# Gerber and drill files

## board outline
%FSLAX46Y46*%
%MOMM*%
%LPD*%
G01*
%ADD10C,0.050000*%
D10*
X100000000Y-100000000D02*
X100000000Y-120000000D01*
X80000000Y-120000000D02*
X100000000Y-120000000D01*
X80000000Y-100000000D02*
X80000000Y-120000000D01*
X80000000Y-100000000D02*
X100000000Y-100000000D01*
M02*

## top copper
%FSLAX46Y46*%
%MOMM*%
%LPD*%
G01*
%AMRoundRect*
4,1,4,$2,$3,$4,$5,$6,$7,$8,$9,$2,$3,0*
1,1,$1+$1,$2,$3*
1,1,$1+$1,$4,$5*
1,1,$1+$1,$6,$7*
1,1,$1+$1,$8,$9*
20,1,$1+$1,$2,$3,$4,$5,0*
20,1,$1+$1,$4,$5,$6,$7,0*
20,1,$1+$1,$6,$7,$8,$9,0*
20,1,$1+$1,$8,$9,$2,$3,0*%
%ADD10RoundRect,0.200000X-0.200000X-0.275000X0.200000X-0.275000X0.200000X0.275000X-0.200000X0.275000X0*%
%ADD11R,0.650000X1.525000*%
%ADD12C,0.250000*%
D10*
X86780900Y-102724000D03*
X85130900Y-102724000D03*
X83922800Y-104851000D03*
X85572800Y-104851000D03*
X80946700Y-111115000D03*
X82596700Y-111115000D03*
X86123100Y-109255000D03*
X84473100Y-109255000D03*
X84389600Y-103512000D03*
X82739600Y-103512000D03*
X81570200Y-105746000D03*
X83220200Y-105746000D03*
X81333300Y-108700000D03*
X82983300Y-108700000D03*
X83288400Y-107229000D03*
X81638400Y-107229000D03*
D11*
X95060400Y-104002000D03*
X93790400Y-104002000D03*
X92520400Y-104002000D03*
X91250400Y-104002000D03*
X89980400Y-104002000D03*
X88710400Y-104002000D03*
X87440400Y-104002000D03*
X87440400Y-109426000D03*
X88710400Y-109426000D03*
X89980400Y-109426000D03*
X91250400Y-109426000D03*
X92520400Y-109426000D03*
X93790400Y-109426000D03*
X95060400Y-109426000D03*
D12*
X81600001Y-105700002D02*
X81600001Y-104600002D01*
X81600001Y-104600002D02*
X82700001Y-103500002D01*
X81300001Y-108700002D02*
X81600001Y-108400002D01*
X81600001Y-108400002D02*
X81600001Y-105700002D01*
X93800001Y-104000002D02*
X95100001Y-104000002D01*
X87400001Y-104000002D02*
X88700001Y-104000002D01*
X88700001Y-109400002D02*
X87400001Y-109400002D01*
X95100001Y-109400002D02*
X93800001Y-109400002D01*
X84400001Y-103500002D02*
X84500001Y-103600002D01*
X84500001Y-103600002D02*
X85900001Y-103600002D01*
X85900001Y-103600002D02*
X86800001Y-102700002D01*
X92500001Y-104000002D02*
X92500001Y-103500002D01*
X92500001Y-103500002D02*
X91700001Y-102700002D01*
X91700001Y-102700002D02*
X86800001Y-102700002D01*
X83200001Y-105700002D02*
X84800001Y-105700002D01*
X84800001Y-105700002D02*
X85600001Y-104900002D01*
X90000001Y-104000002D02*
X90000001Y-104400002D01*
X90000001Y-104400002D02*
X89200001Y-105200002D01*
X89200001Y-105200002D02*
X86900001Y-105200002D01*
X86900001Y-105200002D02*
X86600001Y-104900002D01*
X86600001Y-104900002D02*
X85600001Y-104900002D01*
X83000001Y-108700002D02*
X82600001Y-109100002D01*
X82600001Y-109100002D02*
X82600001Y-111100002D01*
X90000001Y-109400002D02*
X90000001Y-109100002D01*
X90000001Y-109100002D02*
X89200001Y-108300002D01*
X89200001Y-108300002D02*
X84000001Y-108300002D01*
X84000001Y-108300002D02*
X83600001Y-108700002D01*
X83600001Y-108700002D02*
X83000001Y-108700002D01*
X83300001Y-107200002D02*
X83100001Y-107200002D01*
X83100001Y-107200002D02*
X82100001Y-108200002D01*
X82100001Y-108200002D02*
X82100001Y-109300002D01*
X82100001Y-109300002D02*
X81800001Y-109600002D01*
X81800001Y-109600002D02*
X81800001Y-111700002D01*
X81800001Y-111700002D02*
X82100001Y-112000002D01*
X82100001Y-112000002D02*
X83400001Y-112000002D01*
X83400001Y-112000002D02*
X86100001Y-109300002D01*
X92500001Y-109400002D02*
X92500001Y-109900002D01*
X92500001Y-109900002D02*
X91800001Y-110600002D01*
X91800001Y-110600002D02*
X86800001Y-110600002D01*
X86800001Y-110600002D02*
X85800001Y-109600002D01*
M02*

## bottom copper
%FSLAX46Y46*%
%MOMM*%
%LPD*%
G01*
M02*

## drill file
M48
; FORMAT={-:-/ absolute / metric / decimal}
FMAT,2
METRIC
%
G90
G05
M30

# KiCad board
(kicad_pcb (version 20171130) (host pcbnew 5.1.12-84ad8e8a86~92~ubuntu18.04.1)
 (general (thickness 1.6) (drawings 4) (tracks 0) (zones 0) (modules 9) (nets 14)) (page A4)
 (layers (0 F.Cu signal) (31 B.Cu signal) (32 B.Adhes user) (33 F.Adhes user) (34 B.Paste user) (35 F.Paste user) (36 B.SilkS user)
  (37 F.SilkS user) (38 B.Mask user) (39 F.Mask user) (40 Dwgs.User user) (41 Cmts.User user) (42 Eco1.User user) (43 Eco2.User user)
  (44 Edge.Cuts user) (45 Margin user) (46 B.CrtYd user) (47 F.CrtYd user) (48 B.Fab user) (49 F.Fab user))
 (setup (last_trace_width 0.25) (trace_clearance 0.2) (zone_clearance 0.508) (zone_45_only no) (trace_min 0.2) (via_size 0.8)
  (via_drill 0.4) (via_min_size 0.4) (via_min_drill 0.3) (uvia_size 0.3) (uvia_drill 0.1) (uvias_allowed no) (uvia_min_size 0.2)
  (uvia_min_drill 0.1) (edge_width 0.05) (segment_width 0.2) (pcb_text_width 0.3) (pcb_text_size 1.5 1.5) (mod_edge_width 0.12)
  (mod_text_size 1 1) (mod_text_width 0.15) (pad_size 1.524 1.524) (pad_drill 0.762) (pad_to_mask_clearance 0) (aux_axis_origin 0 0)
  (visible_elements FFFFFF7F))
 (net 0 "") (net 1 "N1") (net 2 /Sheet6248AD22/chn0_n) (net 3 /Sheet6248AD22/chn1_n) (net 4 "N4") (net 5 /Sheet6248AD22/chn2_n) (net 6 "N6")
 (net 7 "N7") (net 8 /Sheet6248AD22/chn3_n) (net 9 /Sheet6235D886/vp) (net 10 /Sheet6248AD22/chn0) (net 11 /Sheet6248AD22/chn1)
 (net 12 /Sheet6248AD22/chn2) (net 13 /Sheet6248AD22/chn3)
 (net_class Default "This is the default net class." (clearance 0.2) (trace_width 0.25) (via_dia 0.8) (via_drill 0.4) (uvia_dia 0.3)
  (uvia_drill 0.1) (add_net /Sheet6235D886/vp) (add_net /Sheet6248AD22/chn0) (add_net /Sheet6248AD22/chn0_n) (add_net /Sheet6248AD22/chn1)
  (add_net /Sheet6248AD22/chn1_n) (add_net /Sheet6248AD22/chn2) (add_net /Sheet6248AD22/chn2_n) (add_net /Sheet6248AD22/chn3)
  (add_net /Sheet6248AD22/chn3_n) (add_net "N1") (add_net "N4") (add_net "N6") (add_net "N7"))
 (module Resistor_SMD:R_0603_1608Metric (layer F.Cu) (at 85.955900 102.724000)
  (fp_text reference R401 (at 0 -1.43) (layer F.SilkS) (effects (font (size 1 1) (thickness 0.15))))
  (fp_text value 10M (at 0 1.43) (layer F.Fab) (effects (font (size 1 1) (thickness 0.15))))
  (pad 2 smd roundrect (at 0.825 0) (size 0.8 0.95) (layers F.Cu F.Mask F.Paste) (roundrect_rratio 0.25) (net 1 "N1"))
  (pad 1 smd roundrect (at -0.825 0) (size 0.8 0.95) (layers F.Cu F.Mask F.Paste) (roundrect_rratio 0.25) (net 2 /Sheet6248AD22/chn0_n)))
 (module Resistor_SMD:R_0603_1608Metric (layer F.Cu) (at 84.747800 104.851000)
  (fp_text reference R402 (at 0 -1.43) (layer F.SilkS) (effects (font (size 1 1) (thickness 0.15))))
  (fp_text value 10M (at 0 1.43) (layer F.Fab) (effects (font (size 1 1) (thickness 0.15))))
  (pad 1 smd roundrect (at -0.825 0) (size 0.8 0.95) (layers F.Cu F.Mask F.Paste) (roundrect_rratio 0.25) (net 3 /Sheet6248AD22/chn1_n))
  (pad 2 smd roundrect (at 0.825 0) (size 0.8 0.95) (layers F.Cu F.Mask F.Paste) (roundrect_rratio 0.25) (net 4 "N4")))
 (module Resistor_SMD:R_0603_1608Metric (layer F.Cu) (at 81.771700 111.115000)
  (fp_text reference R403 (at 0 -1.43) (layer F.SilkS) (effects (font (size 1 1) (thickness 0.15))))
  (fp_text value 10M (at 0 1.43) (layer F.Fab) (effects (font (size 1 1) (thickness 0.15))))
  (pad 1 smd roundrect (at -0.825 0) (size 0.8 0.95) (layers F.Cu F.Mask F.Paste) (roundrect_rratio 0.25) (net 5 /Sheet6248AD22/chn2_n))
  (pad 2 smd roundrect (at 0.825 0) (size 0.8 0.95) (layers F.Cu F.Mask F.Paste) (roundrect_rratio 0.25) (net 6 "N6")))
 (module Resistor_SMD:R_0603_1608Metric (layer F.Cu) (at 85.298100 109.255000)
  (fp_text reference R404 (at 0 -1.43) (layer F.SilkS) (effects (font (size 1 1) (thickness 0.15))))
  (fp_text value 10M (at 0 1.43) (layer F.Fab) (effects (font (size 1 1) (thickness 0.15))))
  (pad 2 smd roundrect (at 0.825 0) (size 0.8 0.95) (layers F.Cu F.Mask F.Paste) (roundrect_rratio 0.25) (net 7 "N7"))
  (pad 1 smd roundrect (at -0.825 0) (size 0.8 0.95) (layers F.Cu F.Mask F.Paste) (roundrect_rratio 0.25) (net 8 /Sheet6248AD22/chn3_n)))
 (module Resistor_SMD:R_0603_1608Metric (layer F.Cu) (at 83.564600 103.512000)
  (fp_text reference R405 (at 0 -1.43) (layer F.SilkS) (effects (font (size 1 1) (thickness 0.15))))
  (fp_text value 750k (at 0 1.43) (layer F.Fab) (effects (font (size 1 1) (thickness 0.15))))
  (pad 2 smd roundrect (at 0.825 0) (size 0.8 0.95) (layers F.Cu F.Mask F.Paste) (roundrect_rratio 0.25) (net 1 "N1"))
  (pad 1 smd roundrect (at -0.825 0) (size 0.8 0.95) (layers F.Cu F.Mask F.Paste) (roundrect_rratio 0.25) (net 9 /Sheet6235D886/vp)))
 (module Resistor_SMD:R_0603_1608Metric (layer F.Cu) (at 82.395200 105.746000)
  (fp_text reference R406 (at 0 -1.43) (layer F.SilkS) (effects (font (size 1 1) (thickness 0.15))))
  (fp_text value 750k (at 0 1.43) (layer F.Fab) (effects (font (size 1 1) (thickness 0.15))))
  (pad 1 smd roundrect (at -0.825 0) (size 0.8 0.95) (layers F.Cu F.Mask F.Paste) (roundrect_rratio 0.25) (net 9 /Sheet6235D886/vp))
  (pad 2 smd roundrect (at 0.825 0) (size 0.8 0.95) (layers F.Cu F.Mask F.Paste) (roundrect_rratio 0.25) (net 4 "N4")))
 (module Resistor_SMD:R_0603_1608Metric (layer F.Cu) (at 82.158300 108.700000)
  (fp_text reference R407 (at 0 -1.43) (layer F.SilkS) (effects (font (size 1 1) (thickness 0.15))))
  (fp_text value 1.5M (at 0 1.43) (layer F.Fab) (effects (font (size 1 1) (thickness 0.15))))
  (pad 1 smd roundrect (at -0.825 0) (size 0.8 0.95) (layers F.Cu F.Mask F.Paste) (roundrect_rratio 0.25) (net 9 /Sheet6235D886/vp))
  (pad 2 smd roundrect (at 0.825 0) (size 0.8 0.95) (layers F.Cu F.Mask F.Paste) (roundrect_rratio 0.25) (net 6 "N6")))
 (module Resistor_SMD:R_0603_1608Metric (layer F.Cu) (at 82.463400 107.229000)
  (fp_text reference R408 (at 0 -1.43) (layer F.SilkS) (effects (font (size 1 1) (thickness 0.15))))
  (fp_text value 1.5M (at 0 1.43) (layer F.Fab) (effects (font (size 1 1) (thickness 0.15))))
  (pad 2 smd roundrect (at 0.825 0) (size 0.8 0.95) (layers F.Cu F.Mask F.Paste) (roundrect_rratio 0.25) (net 7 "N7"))
  (pad 1 smd roundrect (at -0.825 0) (size 0.8 0.95) (layers F.Cu F.Mask F.Paste) (roundrect_rratio 0.25) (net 9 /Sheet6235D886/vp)))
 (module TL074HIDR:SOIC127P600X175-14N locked (layer F.Cu) (at 91.250400 106.714000 270.000000)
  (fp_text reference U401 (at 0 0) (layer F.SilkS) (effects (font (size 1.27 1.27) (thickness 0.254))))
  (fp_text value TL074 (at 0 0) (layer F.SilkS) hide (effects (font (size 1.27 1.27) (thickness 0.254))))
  (pad 1 smd rect (at -2.712 -3.81) (size 0.65 1.525) (layers F.Cu F.Mask F.Paste) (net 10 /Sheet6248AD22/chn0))
  (pad 2 smd rect (at -2.712 -2.54) (size 0.65 1.525) (layers F.Cu F.Mask F.Paste) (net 10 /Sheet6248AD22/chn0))
  (pad 3 smd rect (at -2.712 -1.27) (size 0.65 1.525) (layers F.Cu F.Mask F.Paste) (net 1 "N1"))
  (pad 4 smd rect (at -2.712 0) (size 0.65 1.525) (layers F.Cu F.Mask F.Paste))
  (pad 5 smd rect (at -2.712 1.27) (size 0.65 1.525) (layers F.Cu F.Mask F.Paste) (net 4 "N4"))
  (pad 6 smd rect (at -2.712 2.54) (size 0.65 1.525) (layers F.Cu F.Mask F.Paste) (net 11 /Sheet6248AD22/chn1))
  (pad 7 smd rect (at -2.712 3.81) (size 0.65 1.525) (layers F.Cu F.Mask F.Paste) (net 11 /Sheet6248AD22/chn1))
  (pad 8 smd rect (at 2.712 3.81) (size 0.65 1.525) (layers F.Cu F.Mask F.Paste) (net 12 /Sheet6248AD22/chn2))
  (pad 9 smd rect (at 2.712 2.54) (size 0.65 1.525) (layers F.Cu F.Mask F.Paste) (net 12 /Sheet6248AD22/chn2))
  (pad 10 smd rect (at 2.712 1.27) (size 0.65 1.525) (layers F.Cu F.Mask F.Paste) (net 6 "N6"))
  (pad 11 smd rect (at 2.712 0) (size 0.65 1.525) (layers F.Cu F.Mask F.Paste))
  (pad 12 smd rect (at 2.712 -1.27) (size 0.65 1.525) (layers F.Cu F.Mask F.Paste) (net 7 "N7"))
  (pad 13 smd rect (at 2.712 -2.54) (size 0.65 1.525) (layers F.Cu F.Mask F.Paste) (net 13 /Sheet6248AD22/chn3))
  (pad 14 smd rect (at 2.712 -3.81) (size 0.65 1.525) (layers F.Cu F.Mask F.Paste) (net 13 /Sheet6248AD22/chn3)))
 (gr_line (start 100 100) (end 100 120) (layer Edge.Cuts) (width 0.05))
 (gr_line (start 80 120) (end 100 120) (layer Edge.Cuts) (width 0.05))
 (gr_line (start 80 100) (end 80 120) (layer Edge.Cuts) (width 0.05))
 (gr_line (start 80 100) (end 100 100) (layer Edge.Cuts) (width 0.05))
 (segment (start 81.600001 105.700002) (end 81.600001 104.600002) (width 0.250000) (layer F.Cu) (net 9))
 (segment (start 81.600001 104.600002) (end 82.700001 103.500002) (width 0.250000) (layer F.Cu) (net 9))
 (segment (start 81.300001 108.700002) (end 81.600001 108.400002) (width 0.250000) (layer F.Cu) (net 9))
 (segment (start 81.600001 108.400002) (end 81.600001 105.700002) (width 0.250000) (layer F.Cu) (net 9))
 (segment (start 93.800001 104.000002) (end 95.100001 104.000002) (width 0.250000) (layer F.Cu) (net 10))
 (segment (start 87.400001 104.000002) (end 88.700001 104.000002) (width 0.250000) (layer F.Cu) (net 11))
 (segment (start 88.700001 109.400002) (end 87.400001 109.400002) (width 0.250000) (layer F.Cu) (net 12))
 (segment (start 95.100001 109.400002) (end 93.800001 109.400002) (width 0.250000) (layer F.Cu) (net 13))
 (segment (start 84.400001 103.500002) (end 84.500001 103.600002) (width 0.250000) (layer F.Cu) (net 1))
 (segment (start 84.500001 103.600002) (end 85.900001 103.600002) (width 0.250000) (layer F.Cu) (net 1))
 (segment (start 85.900001 103.600002) (end 86.800001 102.700002) (width 0.250000) (layer F.Cu) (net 1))
 (segment (start 92.500001 104.000002) (end 92.500001 103.500002) (width 0.250000) (layer F.Cu) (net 1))
 (segment (start 92.500001 103.500002) (end 91.700001 102.700002) (width 0.250000) (layer F.Cu) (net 1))
 (segment (start 91.700001 102.700002) (end 86.800001 102.700002) (width 0.250000) (layer F.Cu) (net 1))
 (segment (start 83.200001 105.700002) (end 84.800001 105.700002) (width 0.250000) (layer F.Cu) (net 4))
 (segment (start 84.800001 105.700002) (end 85.600001 104.900002) (width 0.250000) (layer F.Cu) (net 4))
 (segment (start 90.000001 104.000002) (end 90.000001 104.400002) (width 0.250000) (layer F.Cu) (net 4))
 (segment (start 90.000001 104.400002) (end 89.200001 105.200002) (width 0.250000) (layer F.Cu) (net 4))
 (segment (start 89.200001 105.200002) (end 86.900001 105.200002) (width 0.250000) (layer F.Cu) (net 4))
 (segment (start 86.900001 105.200002) (end 86.600001 104.900002) (width 0.250000) (layer F.Cu) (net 4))
 (segment (start 86.600001 104.900002) (end 85.600001 104.900002) (width 0.250000) (layer F.Cu) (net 4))
 (segment (start 83.000001 108.700002) (end 82.600001 109.100002) (width 0.250000) (layer F.Cu) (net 6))
 (segment (start 82.600001 109.100002) (end 82.600001 111.100002) (width 0.250000) (layer F.Cu) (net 6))
 (segment (start 90.000001 109.400002) (end 90.000001 109.100002) (width 0.250000) (layer F.Cu) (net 6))
 (segment (start 90.000001 109.100002) (end 89.200001 108.300002) (width 0.250000) (layer F.Cu) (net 6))
 (segment (start 89.200001 108.300002) (end 84.000001 108.300002) (width 0.250000) (layer F.Cu) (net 6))
 (segment (start 84.000001 108.300002) (end 83.600001 108.700002) (width 0.250000) (layer F.Cu) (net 6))
 (segment (start 83.600001 108.700002) (end 83.000001 108.700002) (width 0.250000) (layer F.Cu) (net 6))
 (segment (start 83.300001 107.200002) (end 83.100001 107.200002) (width 0.250000) (layer F.Cu) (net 7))
 (segment (start 83.100001 107.200002) (end 82.100001 108.200002) (width 0.250000) (layer F.Cu) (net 7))
 (segment (start 82.100001 108.200002) (end 82.100001 109.300002) (width 0.250000) (layer F.Cu) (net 7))
 (segment (start 82.100001 109.300002) (end 81.800001 109.600002) (width 0.250000) (layer F.Cu) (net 7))
 (segment (start 81.800001 109.600002) (end 81.800001 111.700002) (width 0.250000) (layer F.Cu) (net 7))
 (segment (start 81.800001 111.700002) (end 82.100001 112.000002) (width 0.250000) (layer F.Cu) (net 7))
 (segment (start 82.100001 112.000002) (end 83.400001 112.000002) (width 0.250000) (layer F.Cu) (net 7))
 (segment (start 83.400001 112.000002) (end 86.100001 109.300002) (width 0.250000) (layer F.Cu) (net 7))
 (segment (start 92.500001 109.400002) (end 92.500001 109.900002) (width 0.250000) (layer F.Cu) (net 7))
 (segment (start 92.500001 109.900002) (end 91.800001 110.600002) (width 0.250000) (layer F.Cu) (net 7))
 (segment (start 91.800001 110.600002) (end 86.800001 110.600002) (width 0.250000) (layer F.Cu) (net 7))
 (segment (start 86.800001 110.600002) (end 85.800001 109.600002) (width 0.250000) (layer F.Cu) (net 7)))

